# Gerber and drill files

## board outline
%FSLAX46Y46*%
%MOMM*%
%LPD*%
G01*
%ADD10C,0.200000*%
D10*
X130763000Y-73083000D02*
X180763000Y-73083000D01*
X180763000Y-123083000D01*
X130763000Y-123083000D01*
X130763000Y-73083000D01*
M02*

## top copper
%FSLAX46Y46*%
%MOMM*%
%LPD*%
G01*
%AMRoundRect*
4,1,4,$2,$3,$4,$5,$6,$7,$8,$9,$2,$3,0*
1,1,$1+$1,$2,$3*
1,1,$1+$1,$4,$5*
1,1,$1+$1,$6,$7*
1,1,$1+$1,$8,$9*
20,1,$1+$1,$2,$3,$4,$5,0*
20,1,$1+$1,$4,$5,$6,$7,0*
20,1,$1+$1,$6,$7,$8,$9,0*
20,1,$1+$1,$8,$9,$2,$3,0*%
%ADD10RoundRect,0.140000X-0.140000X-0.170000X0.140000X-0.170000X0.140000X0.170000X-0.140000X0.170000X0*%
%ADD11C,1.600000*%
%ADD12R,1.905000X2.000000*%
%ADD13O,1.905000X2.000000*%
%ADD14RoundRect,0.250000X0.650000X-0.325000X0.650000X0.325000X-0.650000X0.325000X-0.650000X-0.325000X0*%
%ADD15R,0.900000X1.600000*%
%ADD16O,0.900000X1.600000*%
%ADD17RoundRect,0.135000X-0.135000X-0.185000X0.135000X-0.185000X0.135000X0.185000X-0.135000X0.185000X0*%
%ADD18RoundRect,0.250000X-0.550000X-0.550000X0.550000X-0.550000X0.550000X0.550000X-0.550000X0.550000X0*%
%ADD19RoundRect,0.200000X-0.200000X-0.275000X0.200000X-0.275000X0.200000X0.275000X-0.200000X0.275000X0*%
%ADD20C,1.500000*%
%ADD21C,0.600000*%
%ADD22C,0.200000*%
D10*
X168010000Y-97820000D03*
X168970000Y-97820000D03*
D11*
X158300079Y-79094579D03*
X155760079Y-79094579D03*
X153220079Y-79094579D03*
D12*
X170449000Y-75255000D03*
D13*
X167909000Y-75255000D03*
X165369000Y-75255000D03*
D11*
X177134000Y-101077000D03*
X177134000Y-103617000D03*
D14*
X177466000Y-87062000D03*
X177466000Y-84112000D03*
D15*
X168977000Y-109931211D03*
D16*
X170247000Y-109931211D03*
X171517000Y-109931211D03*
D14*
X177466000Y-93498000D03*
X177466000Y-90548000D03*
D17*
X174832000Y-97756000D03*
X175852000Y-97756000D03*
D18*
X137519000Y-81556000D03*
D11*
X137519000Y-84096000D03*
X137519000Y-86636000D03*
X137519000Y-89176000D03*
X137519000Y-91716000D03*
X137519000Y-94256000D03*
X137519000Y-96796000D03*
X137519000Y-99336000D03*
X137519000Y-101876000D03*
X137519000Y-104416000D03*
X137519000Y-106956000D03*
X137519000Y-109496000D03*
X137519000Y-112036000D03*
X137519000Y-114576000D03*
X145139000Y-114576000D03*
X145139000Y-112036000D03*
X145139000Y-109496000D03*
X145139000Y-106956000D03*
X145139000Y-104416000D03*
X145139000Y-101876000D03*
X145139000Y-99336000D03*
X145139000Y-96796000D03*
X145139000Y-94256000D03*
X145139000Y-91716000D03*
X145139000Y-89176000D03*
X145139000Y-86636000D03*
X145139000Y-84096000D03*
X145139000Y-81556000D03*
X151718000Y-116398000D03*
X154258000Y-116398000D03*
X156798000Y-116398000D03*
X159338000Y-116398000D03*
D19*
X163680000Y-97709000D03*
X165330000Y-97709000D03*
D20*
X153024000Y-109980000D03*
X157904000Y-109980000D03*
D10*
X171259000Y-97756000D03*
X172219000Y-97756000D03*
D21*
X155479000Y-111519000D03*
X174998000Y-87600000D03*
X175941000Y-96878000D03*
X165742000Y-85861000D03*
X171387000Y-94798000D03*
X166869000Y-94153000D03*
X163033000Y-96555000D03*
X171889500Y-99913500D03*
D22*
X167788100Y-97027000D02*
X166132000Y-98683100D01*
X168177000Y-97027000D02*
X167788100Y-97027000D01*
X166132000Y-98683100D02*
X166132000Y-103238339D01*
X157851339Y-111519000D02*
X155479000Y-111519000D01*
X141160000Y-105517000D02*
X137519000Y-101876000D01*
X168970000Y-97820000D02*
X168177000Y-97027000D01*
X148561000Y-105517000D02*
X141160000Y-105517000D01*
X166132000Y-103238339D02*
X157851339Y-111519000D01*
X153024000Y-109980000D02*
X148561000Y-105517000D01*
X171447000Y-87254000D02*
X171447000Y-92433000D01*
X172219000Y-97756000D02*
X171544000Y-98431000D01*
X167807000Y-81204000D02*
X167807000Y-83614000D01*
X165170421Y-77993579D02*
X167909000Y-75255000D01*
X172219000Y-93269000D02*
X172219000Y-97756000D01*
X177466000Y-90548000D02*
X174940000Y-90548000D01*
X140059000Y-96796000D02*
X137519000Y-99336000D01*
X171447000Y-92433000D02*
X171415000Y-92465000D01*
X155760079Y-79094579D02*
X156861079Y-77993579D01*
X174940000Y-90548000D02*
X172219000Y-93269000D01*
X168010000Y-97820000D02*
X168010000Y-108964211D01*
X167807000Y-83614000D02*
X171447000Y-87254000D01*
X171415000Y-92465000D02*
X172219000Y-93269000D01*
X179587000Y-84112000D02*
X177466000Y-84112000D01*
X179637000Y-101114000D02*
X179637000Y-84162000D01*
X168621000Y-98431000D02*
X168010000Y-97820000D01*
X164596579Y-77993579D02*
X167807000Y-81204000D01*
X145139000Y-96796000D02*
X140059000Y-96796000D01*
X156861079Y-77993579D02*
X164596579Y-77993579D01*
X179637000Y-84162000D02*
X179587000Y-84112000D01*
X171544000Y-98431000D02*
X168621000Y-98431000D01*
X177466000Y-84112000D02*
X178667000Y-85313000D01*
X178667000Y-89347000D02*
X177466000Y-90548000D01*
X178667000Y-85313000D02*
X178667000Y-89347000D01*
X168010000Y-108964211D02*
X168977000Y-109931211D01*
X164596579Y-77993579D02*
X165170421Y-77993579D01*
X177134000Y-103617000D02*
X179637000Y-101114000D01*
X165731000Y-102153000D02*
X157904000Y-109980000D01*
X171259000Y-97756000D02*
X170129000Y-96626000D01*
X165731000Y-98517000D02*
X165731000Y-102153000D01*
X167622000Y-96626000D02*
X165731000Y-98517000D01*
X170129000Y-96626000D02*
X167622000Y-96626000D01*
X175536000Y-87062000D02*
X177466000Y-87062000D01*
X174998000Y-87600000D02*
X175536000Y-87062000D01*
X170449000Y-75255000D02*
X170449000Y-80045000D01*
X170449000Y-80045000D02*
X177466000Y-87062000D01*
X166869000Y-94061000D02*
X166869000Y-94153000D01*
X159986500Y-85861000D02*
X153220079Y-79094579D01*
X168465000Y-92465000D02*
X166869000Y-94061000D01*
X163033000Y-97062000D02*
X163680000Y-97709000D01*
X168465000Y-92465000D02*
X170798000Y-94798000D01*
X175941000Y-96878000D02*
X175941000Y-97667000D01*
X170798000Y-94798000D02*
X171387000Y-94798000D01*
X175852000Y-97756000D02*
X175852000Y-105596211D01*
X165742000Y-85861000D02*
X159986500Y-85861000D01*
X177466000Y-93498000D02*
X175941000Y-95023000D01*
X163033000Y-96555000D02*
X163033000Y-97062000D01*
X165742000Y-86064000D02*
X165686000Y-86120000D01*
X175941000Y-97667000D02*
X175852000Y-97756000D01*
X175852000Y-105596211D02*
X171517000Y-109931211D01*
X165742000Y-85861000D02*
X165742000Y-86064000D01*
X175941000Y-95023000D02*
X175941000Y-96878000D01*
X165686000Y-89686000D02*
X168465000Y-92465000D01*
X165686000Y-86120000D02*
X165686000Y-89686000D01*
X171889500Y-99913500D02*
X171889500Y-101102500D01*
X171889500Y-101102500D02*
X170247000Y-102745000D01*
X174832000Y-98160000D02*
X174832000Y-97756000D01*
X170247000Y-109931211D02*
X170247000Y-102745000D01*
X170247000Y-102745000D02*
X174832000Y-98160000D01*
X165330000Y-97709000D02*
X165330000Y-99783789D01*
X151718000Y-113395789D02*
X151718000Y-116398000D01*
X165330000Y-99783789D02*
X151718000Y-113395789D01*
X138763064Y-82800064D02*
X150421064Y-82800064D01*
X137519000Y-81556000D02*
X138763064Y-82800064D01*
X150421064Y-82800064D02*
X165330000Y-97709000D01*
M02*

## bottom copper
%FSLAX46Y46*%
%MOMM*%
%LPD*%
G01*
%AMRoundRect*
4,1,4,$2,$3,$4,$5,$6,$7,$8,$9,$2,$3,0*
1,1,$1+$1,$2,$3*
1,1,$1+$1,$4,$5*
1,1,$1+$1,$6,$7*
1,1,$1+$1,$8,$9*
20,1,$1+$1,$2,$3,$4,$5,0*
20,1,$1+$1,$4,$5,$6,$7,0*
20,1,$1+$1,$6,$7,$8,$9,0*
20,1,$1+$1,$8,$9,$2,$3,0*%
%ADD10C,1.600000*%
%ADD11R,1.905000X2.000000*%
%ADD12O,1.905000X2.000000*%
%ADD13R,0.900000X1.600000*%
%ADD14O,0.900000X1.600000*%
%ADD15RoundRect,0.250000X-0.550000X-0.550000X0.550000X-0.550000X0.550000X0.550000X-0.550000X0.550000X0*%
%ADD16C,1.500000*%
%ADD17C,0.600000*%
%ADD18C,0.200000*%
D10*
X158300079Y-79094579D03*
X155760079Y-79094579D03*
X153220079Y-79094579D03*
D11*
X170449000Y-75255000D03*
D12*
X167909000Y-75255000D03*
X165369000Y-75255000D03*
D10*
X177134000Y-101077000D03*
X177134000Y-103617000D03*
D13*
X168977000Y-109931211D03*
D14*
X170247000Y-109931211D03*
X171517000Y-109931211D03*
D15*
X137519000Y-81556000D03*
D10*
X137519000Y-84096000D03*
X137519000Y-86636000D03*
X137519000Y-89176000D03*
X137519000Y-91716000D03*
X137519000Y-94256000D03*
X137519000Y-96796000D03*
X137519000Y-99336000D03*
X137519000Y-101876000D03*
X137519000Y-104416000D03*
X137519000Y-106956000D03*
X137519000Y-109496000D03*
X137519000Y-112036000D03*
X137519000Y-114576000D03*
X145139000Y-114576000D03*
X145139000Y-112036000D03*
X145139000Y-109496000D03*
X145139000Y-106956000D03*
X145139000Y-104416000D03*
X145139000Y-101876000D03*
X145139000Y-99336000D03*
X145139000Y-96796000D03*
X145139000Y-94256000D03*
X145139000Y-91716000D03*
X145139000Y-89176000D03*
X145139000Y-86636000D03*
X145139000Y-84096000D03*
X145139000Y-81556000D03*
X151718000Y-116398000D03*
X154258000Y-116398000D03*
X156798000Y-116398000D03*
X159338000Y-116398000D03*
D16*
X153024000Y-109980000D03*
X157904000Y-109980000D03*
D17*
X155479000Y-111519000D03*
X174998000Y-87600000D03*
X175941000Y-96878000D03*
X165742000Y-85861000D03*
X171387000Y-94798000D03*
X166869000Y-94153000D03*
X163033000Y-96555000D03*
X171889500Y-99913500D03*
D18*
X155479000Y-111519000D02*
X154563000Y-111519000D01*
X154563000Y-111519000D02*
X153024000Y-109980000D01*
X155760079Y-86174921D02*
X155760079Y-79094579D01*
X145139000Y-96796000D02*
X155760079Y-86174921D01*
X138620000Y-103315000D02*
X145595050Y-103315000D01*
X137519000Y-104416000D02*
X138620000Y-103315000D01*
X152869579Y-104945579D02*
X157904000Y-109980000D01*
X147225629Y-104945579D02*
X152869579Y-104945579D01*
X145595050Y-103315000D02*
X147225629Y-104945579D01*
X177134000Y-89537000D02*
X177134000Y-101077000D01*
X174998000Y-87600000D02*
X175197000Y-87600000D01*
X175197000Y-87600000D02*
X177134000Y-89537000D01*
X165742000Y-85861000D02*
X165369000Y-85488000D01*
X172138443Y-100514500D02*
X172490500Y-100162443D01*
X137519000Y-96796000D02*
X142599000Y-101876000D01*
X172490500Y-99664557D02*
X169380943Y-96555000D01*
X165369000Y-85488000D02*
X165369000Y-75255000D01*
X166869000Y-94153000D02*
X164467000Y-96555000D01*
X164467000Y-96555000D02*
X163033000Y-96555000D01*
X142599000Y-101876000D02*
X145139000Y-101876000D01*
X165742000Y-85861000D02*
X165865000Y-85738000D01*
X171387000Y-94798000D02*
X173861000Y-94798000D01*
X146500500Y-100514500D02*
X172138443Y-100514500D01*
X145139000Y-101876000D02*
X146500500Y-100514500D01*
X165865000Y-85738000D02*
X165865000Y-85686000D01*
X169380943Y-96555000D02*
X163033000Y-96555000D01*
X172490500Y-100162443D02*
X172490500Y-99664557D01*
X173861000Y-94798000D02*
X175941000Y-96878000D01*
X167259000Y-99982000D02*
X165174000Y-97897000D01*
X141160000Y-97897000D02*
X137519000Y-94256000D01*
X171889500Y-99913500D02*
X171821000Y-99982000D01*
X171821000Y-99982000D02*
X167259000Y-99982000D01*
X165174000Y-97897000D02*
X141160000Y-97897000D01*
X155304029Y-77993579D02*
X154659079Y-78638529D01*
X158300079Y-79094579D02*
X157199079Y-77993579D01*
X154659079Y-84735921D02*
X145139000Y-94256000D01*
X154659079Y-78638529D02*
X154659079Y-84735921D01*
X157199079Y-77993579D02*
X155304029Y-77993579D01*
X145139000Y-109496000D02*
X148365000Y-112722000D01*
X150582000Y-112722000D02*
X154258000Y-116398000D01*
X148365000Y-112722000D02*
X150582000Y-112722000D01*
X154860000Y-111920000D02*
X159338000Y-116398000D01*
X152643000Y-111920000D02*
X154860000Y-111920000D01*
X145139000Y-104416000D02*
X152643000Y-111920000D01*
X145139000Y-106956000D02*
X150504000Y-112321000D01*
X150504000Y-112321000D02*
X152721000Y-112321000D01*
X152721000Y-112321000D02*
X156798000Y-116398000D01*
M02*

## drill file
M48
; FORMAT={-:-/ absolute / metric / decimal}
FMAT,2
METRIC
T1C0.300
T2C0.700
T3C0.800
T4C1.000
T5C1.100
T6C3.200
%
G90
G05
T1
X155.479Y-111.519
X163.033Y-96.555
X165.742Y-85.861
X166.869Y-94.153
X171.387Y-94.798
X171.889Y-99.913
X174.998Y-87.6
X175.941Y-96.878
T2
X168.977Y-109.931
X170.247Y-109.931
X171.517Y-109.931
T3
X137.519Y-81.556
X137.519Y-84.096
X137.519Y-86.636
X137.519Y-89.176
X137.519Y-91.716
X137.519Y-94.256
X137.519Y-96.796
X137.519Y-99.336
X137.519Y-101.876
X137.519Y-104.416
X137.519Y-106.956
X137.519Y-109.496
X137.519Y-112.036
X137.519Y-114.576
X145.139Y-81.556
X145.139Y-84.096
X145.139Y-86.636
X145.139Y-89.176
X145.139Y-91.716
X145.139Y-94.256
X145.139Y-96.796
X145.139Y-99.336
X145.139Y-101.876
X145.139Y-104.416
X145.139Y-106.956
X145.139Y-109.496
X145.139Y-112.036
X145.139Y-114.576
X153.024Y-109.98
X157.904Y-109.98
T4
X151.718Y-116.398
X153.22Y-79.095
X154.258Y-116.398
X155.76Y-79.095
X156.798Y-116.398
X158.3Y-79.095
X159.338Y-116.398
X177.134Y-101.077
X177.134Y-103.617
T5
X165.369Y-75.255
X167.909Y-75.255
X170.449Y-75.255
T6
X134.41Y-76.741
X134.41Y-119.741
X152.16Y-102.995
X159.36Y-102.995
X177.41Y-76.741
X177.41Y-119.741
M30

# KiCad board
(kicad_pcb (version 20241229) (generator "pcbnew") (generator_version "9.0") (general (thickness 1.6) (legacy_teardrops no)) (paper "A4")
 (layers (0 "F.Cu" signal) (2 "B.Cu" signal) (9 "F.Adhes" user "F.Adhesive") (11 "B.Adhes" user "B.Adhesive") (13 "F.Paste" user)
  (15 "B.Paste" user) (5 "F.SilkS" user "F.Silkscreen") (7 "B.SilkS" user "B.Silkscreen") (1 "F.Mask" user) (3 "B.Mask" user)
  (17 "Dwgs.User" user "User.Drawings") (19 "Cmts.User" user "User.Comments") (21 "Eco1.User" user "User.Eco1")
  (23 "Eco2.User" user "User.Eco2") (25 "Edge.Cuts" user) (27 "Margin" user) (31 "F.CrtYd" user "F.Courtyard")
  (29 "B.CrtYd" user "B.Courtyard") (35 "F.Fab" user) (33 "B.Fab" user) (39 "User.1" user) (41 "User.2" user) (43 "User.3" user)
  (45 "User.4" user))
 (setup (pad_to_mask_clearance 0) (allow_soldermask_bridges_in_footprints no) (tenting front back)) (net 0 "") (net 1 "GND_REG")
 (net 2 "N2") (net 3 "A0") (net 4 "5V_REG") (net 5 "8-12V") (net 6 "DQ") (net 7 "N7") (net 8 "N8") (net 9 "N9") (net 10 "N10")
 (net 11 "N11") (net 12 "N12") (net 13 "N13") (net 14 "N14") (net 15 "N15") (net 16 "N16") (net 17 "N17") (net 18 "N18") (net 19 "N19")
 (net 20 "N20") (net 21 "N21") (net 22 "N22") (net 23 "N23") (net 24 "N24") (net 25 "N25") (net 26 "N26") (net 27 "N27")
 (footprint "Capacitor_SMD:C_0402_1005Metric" (layer "F.Cu") (at 168.49 97.82)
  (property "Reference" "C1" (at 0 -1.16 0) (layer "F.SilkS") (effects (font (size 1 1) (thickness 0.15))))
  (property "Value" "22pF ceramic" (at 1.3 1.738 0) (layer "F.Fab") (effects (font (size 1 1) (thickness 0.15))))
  (pad "1" smd roundrect (at -0.48 0) (size 0.56 0.62) (layers "F.Cu" "F.Mask" "F.Paste") (roundrect_rratio 0.25) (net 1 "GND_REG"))
  (pad "2" smd roundrect (at 0.48 0) (size 0.56 0.62) (layers "F.Cu" "F.Mask" "F.Paste") (roundrect_rratio 0.25) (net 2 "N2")))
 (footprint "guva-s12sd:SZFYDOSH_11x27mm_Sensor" (layer "F.Cu") (at 155.760079 91.494579 180)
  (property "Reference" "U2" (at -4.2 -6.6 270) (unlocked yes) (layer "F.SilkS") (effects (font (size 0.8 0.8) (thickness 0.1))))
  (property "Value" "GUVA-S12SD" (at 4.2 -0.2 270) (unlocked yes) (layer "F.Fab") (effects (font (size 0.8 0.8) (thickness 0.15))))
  (pad "" np_thru_hole circle (at -3.6 -11.5 180) (size 3.2 3.2) (drill 3.2) (layers "*.Cu" "*.Mask"))
  (pad "" np_thru_hole circle (at 3.6 -11.5 180) (size 3.2 3.2) (drill 3.2) (layers "*.Cu" "*.Mask"))
  (pad "1" thru_hole circle (at -2.54 12.4 180) (size 1.6 1.6) (drill 1) (layers "*.Cu" "*.Mask") (remove_unused_layers no) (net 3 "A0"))
  (pad "2" thru_hole circle (at 0 12.4 180) (size 1.6 1.6) (drill 1) (layers "*.Cu" "*.Mask") (remove_unused_layers no) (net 1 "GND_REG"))
  (pad "3" thru_hole circle (at 2.54 12.4 180) (size 1.6 1.6) (drill 1) (layers "*.Cu" "*.Mask") (remove_unused_layers no) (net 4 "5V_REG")))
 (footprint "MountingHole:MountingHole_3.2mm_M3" (layer "F.Cu") (at 134.41 119.741)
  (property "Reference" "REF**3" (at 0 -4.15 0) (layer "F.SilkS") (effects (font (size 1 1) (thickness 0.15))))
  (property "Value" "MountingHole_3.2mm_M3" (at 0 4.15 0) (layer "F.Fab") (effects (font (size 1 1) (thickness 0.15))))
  (pad "" np_thru_hole circle (at 0 0) (size 3.2 3.2) (drill 3.2) (layers "*.Cu" "*.Mask")))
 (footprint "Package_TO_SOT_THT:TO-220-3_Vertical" (layer "F.Cu") (at 170.449 75.255 180)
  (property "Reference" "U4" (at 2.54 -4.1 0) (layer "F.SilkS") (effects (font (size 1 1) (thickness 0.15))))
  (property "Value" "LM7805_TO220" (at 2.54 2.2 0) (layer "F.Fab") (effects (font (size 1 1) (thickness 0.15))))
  (pad "1" thru_hole rect (at 0 0 180) (size 1.905 2) (drill 1.1) (layers "*.Cu" "*.Mask") (remove_unused_layers no) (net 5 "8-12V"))
  (pad "2" thru_hole oval (at 2.54 0 180) (size 1.905 2) (drill 1.1) (layers "*.Cu" "*.Mask") (remove_unused_layers no) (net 1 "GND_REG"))
  (pad "3" thru_hole oval (at 5.08 0 180) (size 1.905 2) (drill 1.1) (layers "*.Cu" "*.Mask") (remove_unused_layers no) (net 4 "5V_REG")))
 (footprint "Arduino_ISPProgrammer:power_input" (layer "F.Cu") (at 177.134 102.317)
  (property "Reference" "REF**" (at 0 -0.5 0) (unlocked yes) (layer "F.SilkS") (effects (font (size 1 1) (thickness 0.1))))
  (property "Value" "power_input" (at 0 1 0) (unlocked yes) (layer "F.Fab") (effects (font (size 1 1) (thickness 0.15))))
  (pad "1" thru_hole circle (at 0 -1.24) (size 1.6 1.6) (drill 1) (layers "*.Cu" "*.Mask") (remove_unused_layers no) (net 5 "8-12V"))
  (pad "2" thru_hole circle (at 0 1.3) (size 1.6 1.6) (drill 1) (layers "*.Cu" "*.Mask") (remove_unused_layers no) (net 1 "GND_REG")))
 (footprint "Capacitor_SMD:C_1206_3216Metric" (layer "F.Cu") (at 177.466 85.587 90)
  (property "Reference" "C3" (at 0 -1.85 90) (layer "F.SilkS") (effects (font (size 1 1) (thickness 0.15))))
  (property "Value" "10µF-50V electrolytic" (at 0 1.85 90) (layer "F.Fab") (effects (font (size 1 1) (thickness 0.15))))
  (pad "1" smd roundrect (at -1.475 0 90) (size 1.15 1.8) (layers "F.Cu" "F.Mask" "F.Paste") (roundrect_rratio 0.217391) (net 5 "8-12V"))
  (pad "2" smd roundrect (at 1.475 0 90) (size 1.15 1.8) (layers "F.Cu" "F.Mask" "F.Paste") (roundrect_rratio 0.217391) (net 1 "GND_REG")))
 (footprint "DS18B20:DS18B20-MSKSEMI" (layer "F.Cu") (at 170.247 109.931211)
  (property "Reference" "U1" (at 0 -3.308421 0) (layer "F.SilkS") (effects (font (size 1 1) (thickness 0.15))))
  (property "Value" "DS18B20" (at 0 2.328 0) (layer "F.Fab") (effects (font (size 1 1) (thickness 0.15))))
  (pad "1" thru_hole rect (at -1.27 0) (size 0.9 1.6) (drill 0.7) (layers "*.Cu" "*.Mask") (remove_unused_layers no) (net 1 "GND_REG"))
  (pad "2" thru_hole oval (at 0 0) (size 0.9 1.6) (drill 0.7) (layers "*.Cu" "*.Mask") (remove_unused_layers no) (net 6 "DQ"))
  (pad "3" thru_hole oval (at 1.27 0) (size 0.9 1.6) (drill 0.7) (layers "*.Cu" "*.Mask") (remove_unused_layers no) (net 4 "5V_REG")))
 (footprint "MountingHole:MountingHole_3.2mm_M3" (layer "F.Cu") (at 177.41 119.741)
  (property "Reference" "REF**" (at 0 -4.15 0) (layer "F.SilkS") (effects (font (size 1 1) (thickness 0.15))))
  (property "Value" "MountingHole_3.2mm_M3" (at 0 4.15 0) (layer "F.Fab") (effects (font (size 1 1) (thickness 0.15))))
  (pad "" np_thru_hole circle (at 0 0) (size 3.2 3.2) (drill 3.2) (layers "*.Cu" "*.Mask")))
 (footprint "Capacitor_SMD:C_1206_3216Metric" (layer "F.Cu") (at 177.466 92.023 90)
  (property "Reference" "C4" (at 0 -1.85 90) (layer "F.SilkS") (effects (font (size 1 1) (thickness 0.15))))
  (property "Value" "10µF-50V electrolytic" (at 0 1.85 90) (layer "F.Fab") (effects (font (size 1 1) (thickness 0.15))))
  (pad "1" smd roundrect (at -1.475 0 90) (size 1.15 1.8) (layers "F.Cu" "F.Mask" "F.Paste") (roundrect_rratio 0.217391) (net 4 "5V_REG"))
  (pad "2" smd roundrect (at 1.475 0 90) (size 1.15 1.8) (layers "F.Cu" "F.Mask" "F.Paste") (roundrect_rratio 0.217391) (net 1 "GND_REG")))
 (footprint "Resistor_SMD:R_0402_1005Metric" (layer "F.Cu") (at 175.342 97.756)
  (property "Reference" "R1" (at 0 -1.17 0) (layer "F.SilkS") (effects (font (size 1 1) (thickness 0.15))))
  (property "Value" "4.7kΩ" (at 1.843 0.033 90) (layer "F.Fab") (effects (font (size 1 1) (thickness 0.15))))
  (pad "1" smd roundrect (at -0.51 0) (size 0.54 0.64) (layers "F.Cu" "F.Mask" "F.Paste") (roundrect_rratio 0.25) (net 6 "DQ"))
  (pad "2" smd roundrect (at 0.51 0) (size 0.54 0.64) (layers "F.Cu" "F.Mask" "F.Paste") (roundrect_rratio 0.25) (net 4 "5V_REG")))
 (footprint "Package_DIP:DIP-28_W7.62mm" (layer "F.Cu") (at 137.519 81.556)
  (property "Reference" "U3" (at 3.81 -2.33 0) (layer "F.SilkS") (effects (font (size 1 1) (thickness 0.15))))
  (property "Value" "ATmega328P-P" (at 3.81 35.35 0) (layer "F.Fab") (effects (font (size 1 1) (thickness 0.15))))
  (pad "1" thru_hole roundrect (at 0 0) (size 1.6 1.6) (drill 0.8) (layers "*.Cu" "*.Mask") (remove_unused_layers no)
   (roundrect_rratio 0.15625) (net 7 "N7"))
  (pad "2" thru_hole circle (at 0 2.54) (size 1.6 1.6) (drill 0.8) (layers "*.Cu" "*.Mask") (remove_unused_layers no) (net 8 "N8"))
  (pad "3" thru_hole circle (at 0 5.08) (size 1.6 1.6) (drill 0.8) (layers "*.Cu" "*.Mask") (remove_unused_layers no) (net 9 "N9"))
  (pad "4" thru_hole circle (at 0 7.62) (size 1.6 1.6) (drill 0.8) (layers "*.Cu" "*.Mask") (remove_unused_layers no) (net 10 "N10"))
  (pad "5" thru_hole circle (at 0 10.16) (size 1.6 1.6) (drill 0.8) (layers "*.Cu" "*.Mask") (remove_unused_layers no) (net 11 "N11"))
  (pad "6" thru_hole circle (at 0 12.7) (size 1.6 1.6) (drill 0.8) (layers "*.Cu" "*.Mask") (remove_unused_layers no) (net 6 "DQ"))
  (pad "7" thru_hole circle (at 0 15.24) (size 1.6 1.6) (drill 0.8) (layers "*.Cu" "*.Mask") (remove_unused_layers no) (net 4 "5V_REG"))
  (pad "8" thru_hole circle (at 0 17.78) (size 1.6 1.6) (drill 0.8) (layers "*.Cu" "*.Mask") (remove_unused_layers no) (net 1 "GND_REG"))
  (pad "9" thru_hole circle (at 0 20.32) (size 1.6 1.6) (drill 0.8) (layers "*.Cu" "*.Mask") (remove_unused_layers no) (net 2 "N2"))
  (pad "10" thru_hole circle (at 0 22.86) (size 1.6 1.6) (drill 0.8) (layers "*.Cu" "*.Mask") (remove_unused_layers no) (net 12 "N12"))
  (pad "11" thru_hole circle (at 0 25.4) (size 1.6 1.6) (drill 0.8) (layers "*.Cu" "*.Mask") (remove_unused_layers no) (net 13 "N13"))
  (pad "12" thru_hole circle (at 0 27.94) (size 1.6 1.6) (drill 0.8) (layers "*.Cu" "*.Mask") (remove_unused_layers no) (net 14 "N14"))
  (pad "13" thru_hole circle (at 0 30.48) (size 1.6 1.6) (drill 0.8) (layers "*.Cu" "*.Mask") (remove_unused_layers no) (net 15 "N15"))
  (pad "14" thru_hole circle (at 0 33.02) (size 1.6 1.6) (drill 0.8) (layers "*.Cu" "*.Mask") (remove_unused_layers no) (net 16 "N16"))
  (pad "15" thru_hole circle (at 7.62 33.02) (size 1.6 1.6) (drill 0.8) (layers "*.Cu" "*.Mask") (remove_unused_layers no) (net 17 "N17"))
  (pad "16" thru_hole circle (at 7.62 30.48) (size 1.6 1.6) (drill 0.8) (layers "*.Cu" "*.Mask") (remove_unused_layers no) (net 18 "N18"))
  (pad "17" thru_hole circle (at 7.62 27.94) (size 1.6 1.6) (drill 0.8) (layers "*.Cu" "*.Mask") (remove_unused_layers no) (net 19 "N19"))
  (pad "18" thru_hole circle (at 7.62 25.4) (size 1.6 1.6) (drill 0.8) (layers "*.Cu" "*.Mask") (remove_unused_layers no) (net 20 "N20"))
  (pad "19" thru_hole circle (at 7.62 22.86) (size 1.6 1.6) (drill 0.8) (layers "*.Cu" "*.Mask") (remove_unused_layers no) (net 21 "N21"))
  (pad "20" thru_hole circle (at 7.62 20.32) (size 1.6 1.6) (drill 0.8) (layers "*.Cu" "*.Mask") (remove_unused_layers no) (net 4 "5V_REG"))
  (pad "21" thru_hole circle (at 7.62 17.78) (size 1.6 1.6) (drill 0.8) (layers "*.Cu" "*.Mask") (remove_unused_layers no) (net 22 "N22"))
  (pad "22" thru_hole circle (at 7.62 15.24) (size 1.6 1.6) (drill 0.8) (layers "*.Cu" "*.Mask") (remove_unused_layers no) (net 1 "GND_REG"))
  (pad "23" thru_hole circle (at 7.62 12.7) (size 1.6 1.6) (drill 0.8) (layers "*.Cu" "*.Mask") (remove_unused_layers no) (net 3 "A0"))
  (pad "24" thru_hole circle (at 7.62 10.16) (size 1.6 1.6) (drill 0.8) (layers "*.Cu" "*.Mask") (remove_unused_layers no) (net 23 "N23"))
  (pad "25" thru_hole circle (at 7.62 7.62) (size 1.6 1.6) (drill 0.8) (layers "*.Cu" "*.Mask") (remove_unused_layers no) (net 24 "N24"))
  (pad "26" thru_hole circle (at 7.62 5.08) (size 1.6 1.6) (drill 0.8) (layers "*.Cu" "*.Mask") (remove_unused_layers no) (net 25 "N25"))
  (pad "27" thru_hole circle (at 7.62 2.54) (size 1.6 1.6) (drill 0.8) (layers "*.Cu" "*.Mask") (remove_unused_layers no) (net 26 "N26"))
  (pad "28" thru_hole circle (at 7.62 0) (size 1.6 1.6) (drill 0.8) (layers "*.Cu" "*.Mask") (remove_unused_layers no) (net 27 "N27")))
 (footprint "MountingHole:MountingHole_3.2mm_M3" (layer "F.Cu") (at 177.41 76.741)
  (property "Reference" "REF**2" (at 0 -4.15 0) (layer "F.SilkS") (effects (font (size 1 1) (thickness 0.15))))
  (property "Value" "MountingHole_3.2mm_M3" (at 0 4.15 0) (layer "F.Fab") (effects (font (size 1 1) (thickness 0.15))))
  (pad "" np_thru_hole circle (at 0 0) (size 3.2 3.2) (drill 3.2) (layers "*.Cu" "*.Mask")))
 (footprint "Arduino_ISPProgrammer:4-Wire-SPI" (layer "F.Cu") (at 155.528 116.398)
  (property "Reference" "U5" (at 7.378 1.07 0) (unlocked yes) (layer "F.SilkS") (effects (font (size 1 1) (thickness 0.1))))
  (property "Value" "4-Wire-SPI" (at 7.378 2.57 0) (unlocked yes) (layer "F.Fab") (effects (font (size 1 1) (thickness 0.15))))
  (pad "10" thru_hole circle (at -3.81 0) (size 1.6 1.6) (drill 1) (layers "*.Cu" "*.Mask") (remove_unused_layers no) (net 7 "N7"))
  (pad "11" thru_hole circle (at -1.27 0) (size 1.6 1.6) (drill 1) (layers "*.Cu" "*.Mask") (remove_unused_layers no) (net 19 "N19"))
  (pad "12" thru_hole circle (at 1.27 0) (size 1.6 1.6) (drill 1) (layers "*.Cu" "*.Mask") (remove_unused_layers no) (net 20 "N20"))
  (pad "13" thru_hole circle (at 3.81 0) (size 1.6 1.6) (drill 1) (layers "*.Cu" "*.Mask") (remove_unused_layers no) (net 21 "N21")))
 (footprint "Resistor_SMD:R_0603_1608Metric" (layer "F.Cu") (at 164.505 97.709)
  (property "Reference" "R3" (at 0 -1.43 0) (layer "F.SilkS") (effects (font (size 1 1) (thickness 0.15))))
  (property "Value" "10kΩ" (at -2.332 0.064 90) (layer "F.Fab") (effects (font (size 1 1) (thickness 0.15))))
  (pad "1" smd roundrect (at -0.825 0) (size 0.8 0.95) (layers "F.Cu" "F.Mask" "F.Paste") (roundrect_rratio 0.25) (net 4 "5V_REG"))
  (pad "2" smd roundrect (at 0.825 0) (size 0.8 0.95) (layers "F.Cu" "F.Mask" "F.Paste") (roundrect_rratio 0.25) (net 7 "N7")))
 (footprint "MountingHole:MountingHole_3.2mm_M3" (layer "F.Cu") (at 134.41 76.741)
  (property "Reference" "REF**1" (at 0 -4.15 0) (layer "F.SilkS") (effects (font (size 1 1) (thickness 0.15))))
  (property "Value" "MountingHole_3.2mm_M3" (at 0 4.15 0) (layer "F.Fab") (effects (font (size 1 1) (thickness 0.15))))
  (pad "" np_thru_hole circle (at 0 0) (size 3.2 3.2) (drill 3.2) (layers "*.Cu" "*.Mask")))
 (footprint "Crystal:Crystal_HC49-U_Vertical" (layer "F.Cu") (at 153.024 109.98)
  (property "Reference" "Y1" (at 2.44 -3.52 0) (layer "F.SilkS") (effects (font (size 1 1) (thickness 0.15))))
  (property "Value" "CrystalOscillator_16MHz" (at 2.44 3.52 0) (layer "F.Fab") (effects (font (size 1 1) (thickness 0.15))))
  (pad "1" thru_hole circle (at 0 0) (size 1.5 1.5) (drill 0.8) (layers "*.Cu" "*.Mask") (remove_unused_layers no) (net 2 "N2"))
  (pad "2" thru_hole circle (at 4.88 0) (size 1.5 1.5) (drill 0.8) (layers "*.Cu" "*.Mask") (remove_unused_layers no) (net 12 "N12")))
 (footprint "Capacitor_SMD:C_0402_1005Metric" (layer "F.Cu") (at 171.739 97.756)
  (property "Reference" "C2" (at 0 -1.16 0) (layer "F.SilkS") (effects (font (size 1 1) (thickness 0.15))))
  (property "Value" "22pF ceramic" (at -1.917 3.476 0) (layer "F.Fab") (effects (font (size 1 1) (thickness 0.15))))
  (pad "1" smd roundrect (at -0.48 0) (size 0.56 0.62) (layers "F.Cu" "F.Mask" "F.Paste") (roundrect_rratio 0.25) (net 12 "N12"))
  (pad "2" smd roundrect (at 0.48 0) (size 0.56 0.62) (layers "F.Cu" "F.Mask" "F.Paste") (roundrect_rratio 0.25) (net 1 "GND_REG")))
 (gr_rect (start 130.763 73.083) (end 180.763 123.083) (stroke (width 0.2) (type solid)) (fill no) (layer "Edge.Cuts"))
 (segment (start 167.7881 97.027) (end 166.132 98.6831) (width 0.2) (layer "F.Cu") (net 2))
 (segment (start 168.177 97.027) (end 167.7881 97.027) (width 0.2) (layer "F.Cu") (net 2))
 (segment (start 166.132 98.6831) (end 166.132 103.238339) (width 0.2) (layer "F.Cu") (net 2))
 (segment (start 157.851339 111.519) (end 155.479 111.519) (width 0.2) (layer "F.Cu") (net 2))
 (segment (start 141.16 105.517) (end 137.519 101.876) (width 0.2) (layer "F.Cu") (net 2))
 (segment (start 168.97 97.82) (end 168.177 97.027) (width 0.2) (layer "F.Cu") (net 2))
 (segment (start 148.561 105.517) (end 141.16 105.517) (width 0.2) (layer "F.Cu") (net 2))
 (segment (start 166.132 103.238339) (end 157.851339 111.519) (width 0.2) (layer "F.Cu") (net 2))
 (segment (start 153.024 109.98) (end 148.561 105.517) (width 0.2) (layer "F.Cu") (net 2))
 (via (at 155.479 111.519) (size 0.6) (drill 0.3) (layers "F.Cu" "B.Cu") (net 2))
 (segment (start 155.479 111.519) (end 154.563 111.519) (width 0.2) (layer "B.Cu") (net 2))
 (segment (start 154.563 111.519) (end 153.024 109.98) (width 0.2) (layer "B.Cu") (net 2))
 (segment (start 171.447 87.254) (end 171.447 92.433) (width 0.2) (layer "F.Cu") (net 1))
 (segment (start 172.219 97.756) (end 171.544 98.431) (width 0.2) (layer "F.Cu") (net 1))
 (segment (start 167.807 81.204) (end 167.807 83.614) (width 0.2) (layer "F.Cu") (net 1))
 (segment (start 165.170421 77.993579) (end 167.909 75.255) (width 0.2) (layer "F.Cu") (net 1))
 (segment (start 172.219 93.269) (end 172.219 97.756) (width 0.2) (layer "F.Cu") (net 1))
 (segment (start 177.466 90.548) (end 174.94 90.548) (width 0.2) (layer "F.Cu") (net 1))
 (segment (start 140.059 96.796) (end 137.519 99.336) (width 0.2) (layer "F.Cu") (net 1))
 (segment (start 171.447 92.433) (end 171.415 92.465) (width 0.2) (layer "F.Cu") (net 1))
 (segment (start 155.760079 79.094579) (end 156.861079 77.993579) (width 0.2) (layer "F.Cu") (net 1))
 (segment (start 174.94 90.548) (end 172.219 93.269) (width 0.2) (layer "F.Cu") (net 1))
 (segment (start 168.01 97.82) (end 168.01 108.964211) (width 0.2) (layer "F.Cu") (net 1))
 (segment (start 167.807 83.614) (end 171.447 87.254) (width 0.2) (layer "F.Cu") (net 1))
 (segment (start 171.415 92.465) (end 172.219 93.269) (width 0.2) (layer "F.Cu") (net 1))
 (segment (start 179.587 84.112) (end 177.466 84.112) (width 0.2) (layer "F.Cu") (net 1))
 (segment (start 179.637 101.114) (end 179.637 84.162) (width 0.2) (layer "F.Cu") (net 1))
 (segment (start 168.621 98.431) (end 168.01 97.82) (width 0.2) (layer "F.Cu") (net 1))
 (segment (start 164.596579 77.993579) (end 167.807 81.204) (width 0.2) (layer "F.Cu") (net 1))
 (segment (start 145.139 96.796) (end 140.059 96.796) (width 0.2) (layer "F.Cu") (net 1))
 (segment (start 156.861079 77.993579) (end 164.596579 77.993579) (width 0.2) (layer "F.Cu") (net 1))
 (segment (start 179.637 84.162) (end 179.587 84.112) (width 0.2) (layer "F.Cu") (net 1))
 (segment (start 171.544 98.431) (end 168.621 98.431) (width 0.2) (layer "F.Cu") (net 1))
 (segment (start 177.466 84.112) (end 178.667 85.313) (width 0.2) (layer "F.Cu") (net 1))
 (segment (start 178.667 89.347) (end 177.466 90.548) (width 0.2) (layer "F.Cu") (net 1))
 (segment (start 178.667 85.313) (end 178.667 89.347) (width 0.2) (layer "F.Cu") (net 1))
 (segment (start 168.01 108.964211) (end 168.977 109.931211) (width 0.2) (layer "F.Cu") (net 1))
 (segment (start 164.596579 77.993579) (end 165.170421 77.993579) (width 0.2) (layer "F.Cu") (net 1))
 (segment (start 177.134 103.617) (end 179.637 101.114) (width 0.2) (layer "F.Cu") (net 1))
 (segment (start 155.760079 86.174921) (end 155.760079 79.094579) (width 0.2) (layer "B.Cu") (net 1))
 (segment (start 145.139 96.796) (end 155.760079 86.174921) (width 0.2) (layer "B.Cu") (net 1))
 (segment (start 165.731 102.153) (end 157.904 109.98) (width 0.2) (layer "F.Cu") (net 12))
 (segment (start 171.259 97.756) (end 170.129 96.626) (width 0.2) (layer "F.Cu") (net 12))
 (segment (start 165.731 98.517) (end 165.731 102.153) (width 0.2) (layer "F.Cu") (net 12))
 (segment (start 167.622 96.626) (end 165.731 98.517) (width 0.2) (layer "F.Cu") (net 12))
 (segment (start 170.129 96.626) (end 167.622 96.626) (width 0.2) (layer "F.Cu") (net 12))
 (segment (start 138.62 103.315) (end 145.59505 103.315) (width 0.2) (layer "B.Cu") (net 12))
 (segment (start 137.519 104.416) (end 138.62 103.315) (width 0.2) (layer "B.Cu") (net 12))
 (segment (start 152.869579 104.945579) (end 157.904 109.98) (width 0.2) (layer "B.Cu") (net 12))
 (segment (start 147.225629 104.945579) (end 152.869579 104.945579) (width 0.2) (layer "B.Cu") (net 12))
 (segment (start 145.59505 103.315) (end 147.225629 104.945579) (width 0.2) (layer "B.Cu") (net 12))
 (segment (start 175.536 87.062) (end 177.466 87.062) (width 0.2) (layer "F.Cu") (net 5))
 (segment (start 174.998 87.6) (end 175.536 87.062) (width 0.2) (layer "F.Cu") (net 5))
 (segment (start 170.449 75.255) (end 170.449 80.045) (width 0.2) (layer "F.Cu") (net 5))
 (segment (start 170.449 80.045) (end 177.466 87.062) (width 0.2) (layer "F.Cu") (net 5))
 (via (at 174.998 87.6) (size 0.6) (drill 0.3) (layers "F.Cu" "B.Cu") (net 5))
 (segment (start 177.134 89.537) (end 177.134 101.077) (width 0.2) (layer "B.Cu") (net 5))
 (segment (start 174.998 87.6) (end 175.197 87.6) (width 0.2) (layer "B.Cu") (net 5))
 (segment (start 175.197 87.6) (end 177.134 89.537) (width 0.2) (layer "B.Cu") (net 5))
 (segment (start 166.869 94.061) (end 166.869 94.153) (width 0.2) (layer "F.Cu") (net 4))
 (segment (start 159.9865 85.861) (end 153.220079 79.094579) (width 0.2) (layer "F.Cu") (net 4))
 (segment (start 168.465 92.465) (end 166.869 94.061) (width 0.2) (layer "F.Cu") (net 4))
 (segment (start 163.033 97.062) (end 163.68 97.709) (width 0.2) (layer "F.Cu") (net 4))
 (segment (start 168.465 92.465) (end 170.798 94.798) (width 0.2) (layer "F.Cu") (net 4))
 (segment (start 175.941 96.878) (end 175.941 97.667) (width 0.2) (layer "F.Cu") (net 4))
 (segment (start 170.798 94.798) (end 171.387 94.798) (width 0.2) (layer "F.Cu") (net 4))
 (segment (start 175.852 97.756) (end 175.852 105.596211) (width 0.2) (layer "F.Cu") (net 4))
 (segment (start 165.742 85.861) (end 159.9865 85.861) (width 0.2) (layer "F.Cu") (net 4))
 (segment (start 177.466 93.498) (end 175.941 95.023) (width 0.2) (layer "F.Cu") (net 4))
 (segment (start 163.033 96.555) (end 163.033 97.062) (width 0.2) (layer "F.Cu") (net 4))
 (segment (start 165.742 86.064) (end 165.686 86.12) (width 0.2) (layer "F.Cu") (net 4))
 (segment (start 175.941 97.667) (end 175.852 97.756) (width 0.2) (layer "F.Cu") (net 4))
 (segment (start 175.852 105.596211) (end 171.517 109.931211) (width 0.2) (layer "F.Cu") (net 4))
 (segment (start 165.742 85.861) (end 165.742 86.064) (width 0.2) (layer "F.Cu") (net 4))
 (segment (start 175.941 95.023) (end 175.941 96.878) (width 0.2) (layer "F.Cu") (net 4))
 (segment (start 165.686 89.686) (end 168.465 92.465) (width 0.2) (layer "F.Cu") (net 4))
 (segment (start 165.686 86.12) (end 165.686 89.686) (width 0.2) (layer "F.Cu") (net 4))
 (via (at 175.941 96.878) (size 0.6) (drill 0.3) (layers "F.Cu" "B.Cu") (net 4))
 (via (at 165.742 85.861) (size 0.6) (drill 0.3) (layers "F.Cu" "B.Cu") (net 4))
 (via (at 171.387 94.798) (size 0.6) (drill 0.3) (layers "F.Cu" "B.Cu") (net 4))
 (via (at 166.869 94.153) (size 0.6) (drill 0.3) (layers "F.Cu" "B.Cu") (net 4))
 (via (at 163.033 96.555) (size 0.6) (drill 0.3) (layers "F.Cu" "B.Cu") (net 4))
 (segment (start 165.742 85.861) (end 165.369 85.488) (width 0.2) (layer "B.Cu") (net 4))
 (segment (start 172.138443 100.5145) (end 172.4905 100.162443) (width 0.2) (layer "B.Cu") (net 4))
 (segment (start 137.519 96.796) (end 142.599 101.876) (width 0.2) (layer "B.Cu") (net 4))
 (segment (start 172.4905 99.664557) (end 169.380943 96.555) (width 0.2) (layer "B.Cu") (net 4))
 (segment (start 165.369 85.488) (end 165.369 75.255) (width 0.2) (layer "B.Cu") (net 4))
 (segment (start 166.869 94.153) (end 164.467 96.555) (width 0.2) (layer "B.Cu") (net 4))
 (segment (start 164.467 96.555) (end 163.033 96.555) (width 0.2) (layer "B.Cu") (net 4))
 (segment (start 142.599 101.876) (end 145.139 101.876) (width 0.2) (layer "B.Cu") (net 4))
 (segment (start 165.742 85.861) (end 165.865 85.738) (width 0.2) (layer "B.Cu") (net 4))
 (segment (start 171.387 94.798) (end 173.861 94.798) (width 0.2) (layer "B.Cu") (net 4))
 (segment (start 146.5005 100.5145) (end 172.138443 100.5145) (width 0.2) (layer "B.Cu") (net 4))
 (segment (start 145.139 101.876) (end 146.5005 100.5145) (width 0.2) (layer "B.Cu") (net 4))
 (segment (start 165.865 85.738) (end 165.865 85.686) (width 0.2) (layer "B.Cu") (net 4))
 (segment (start 169.380943 96.555) (end 163.033 96.555) (width 0.2) (layer "B.Cu") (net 4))
 (segment (start 172.4905 100.162443) (end 172.4905 99.664557) (width 0.2) (layer "B.Cu") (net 4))
 (segment (start 173.861 94.798) (end 175.941 96.878) (width 0.2) (layer "B.Cu") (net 4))
 (segment (start 171.8895 99.9135) (end 171.8895 101.1025) (width 0.2) (layer "F.Cu") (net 6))
 (segment (start 171.8895 101.1025) (end 170.247 102.745) (width 0.2) (layer "F.Cu") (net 6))
 (segment (start 174.832 98.16) (end 174.832 97.756) (width 0.2) (layer "F.Cu") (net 6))
 (segment (start 170.247 109.931211) (end 170.247 102.745) (width 0.2) (layer "F.Cu") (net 6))
 (segment (start 170.247 102.745) (end 174.832 98.16) (width 0.2) (layer "F.Cu") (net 6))
 (via (at 171.8895 99.9135) (size 0.6) (drill 0.3) (layers "F.Cu" "B.Cu") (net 6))
 (segment (start 167.259 99.982) (end 165.174 97.897) (width 0.2) (layer "B.Cu") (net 6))
 (segment (start 141.16 97.897) (end 137.519 94.256) (width 0.2) (layer "B.Cu") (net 6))
 (segment (start 171.8895 99.9135) (end 171.821 99.982) (width 0.2) (layer "B.Cu") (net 6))
 (segment (start 171.821 99.982) (end 167.259 99.982) (width 0.2) (layer "B.Cu") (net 6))
 (segment (start 165.174 97.897) (end 141.16 97.897) (width 0.2) (layer "B.Cu") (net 6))
 (segment (start 165.33 97.709) (end 165.33 99.783789) (width 0.2) (layer "F.Cu") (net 7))
 (segment (start 151.718 113.395789) (end 151.718 116.398) (width 0.2) (layer "F.Cu") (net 7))
 (segment (start 165.33 99.783789) (end 151.718 113.395789) (width 0.2) (layer "F.Cu") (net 7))
 (segment (start 138.763064 82.800064) (end 150.421064 82.800064) (width 0.2) (layer "F.Cu") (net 7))
 (segment (start 137.519 81.556) (end 138.763064 82.800064) (width 0.2) (layer "F.Cu") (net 7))
 (segment (start 150.421064 82.800064) (end 165.33 97.709) (width 0.2) (layer "F.Cu") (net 7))
 (segment (start 155.304029 77.993579) (end 154.659079 78.638529) (width 0.2) (layer "B.Cu") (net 3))
 (segment (start 158.300079 79.094579) (end 157.199079 77.993579) (width 0.2) (layer "B.Cu") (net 3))
 (segment (start 154.659079 84.735921) (end 145.139 94.256) (width 0.2) (layer "B.Cu") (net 3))
 (segment (start 154.659079 78.638529) (end 154.659079 84.735921) (width 0.2) (layer "B.Cu") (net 3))
 (segment (start 157.199079 77.993579) (end 155.304029 77.993579) (width 0.2) (layer "B.Cu") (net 3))
 (segment (start 145.139 109.496) (end 148.365 112.722) (width 0.2) (layer "B.Cu") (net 19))
 (segment (start 150.582 112.722) (end 154.258 116.398) (width 0.2) (layer "B.Cu") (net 19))
 (segment (start 148.365 112.722) (end 150.582 112.722) (width 0.2) (layer "B.Cu") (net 19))
 (segment (start 154.86 111.92) (end 159.338 116.398) (width 0.2) (layer "B.Cu") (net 21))
 (segment (start 152.643 111.92) (end 154.86 111.92) (width 0.2) (layer "B.Cu") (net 21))
 (segment (start 145.139 104.416) (end 152.643 111.92) (width 0.2) (layer "B.Cu") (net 21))
 (segment (start 145.139 106.956) (end 150.504 112.321) (width 0.2) (layer "B.Cu") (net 20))
 (segment (start 150.504 112.321) (end 152.721 112.321) (width 0.2) (layer "B.Cu") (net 20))
 (segment (start 152.721 112.321) (end 156.798 116.398) (width 0.2) (layer "B.Cu") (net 20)))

